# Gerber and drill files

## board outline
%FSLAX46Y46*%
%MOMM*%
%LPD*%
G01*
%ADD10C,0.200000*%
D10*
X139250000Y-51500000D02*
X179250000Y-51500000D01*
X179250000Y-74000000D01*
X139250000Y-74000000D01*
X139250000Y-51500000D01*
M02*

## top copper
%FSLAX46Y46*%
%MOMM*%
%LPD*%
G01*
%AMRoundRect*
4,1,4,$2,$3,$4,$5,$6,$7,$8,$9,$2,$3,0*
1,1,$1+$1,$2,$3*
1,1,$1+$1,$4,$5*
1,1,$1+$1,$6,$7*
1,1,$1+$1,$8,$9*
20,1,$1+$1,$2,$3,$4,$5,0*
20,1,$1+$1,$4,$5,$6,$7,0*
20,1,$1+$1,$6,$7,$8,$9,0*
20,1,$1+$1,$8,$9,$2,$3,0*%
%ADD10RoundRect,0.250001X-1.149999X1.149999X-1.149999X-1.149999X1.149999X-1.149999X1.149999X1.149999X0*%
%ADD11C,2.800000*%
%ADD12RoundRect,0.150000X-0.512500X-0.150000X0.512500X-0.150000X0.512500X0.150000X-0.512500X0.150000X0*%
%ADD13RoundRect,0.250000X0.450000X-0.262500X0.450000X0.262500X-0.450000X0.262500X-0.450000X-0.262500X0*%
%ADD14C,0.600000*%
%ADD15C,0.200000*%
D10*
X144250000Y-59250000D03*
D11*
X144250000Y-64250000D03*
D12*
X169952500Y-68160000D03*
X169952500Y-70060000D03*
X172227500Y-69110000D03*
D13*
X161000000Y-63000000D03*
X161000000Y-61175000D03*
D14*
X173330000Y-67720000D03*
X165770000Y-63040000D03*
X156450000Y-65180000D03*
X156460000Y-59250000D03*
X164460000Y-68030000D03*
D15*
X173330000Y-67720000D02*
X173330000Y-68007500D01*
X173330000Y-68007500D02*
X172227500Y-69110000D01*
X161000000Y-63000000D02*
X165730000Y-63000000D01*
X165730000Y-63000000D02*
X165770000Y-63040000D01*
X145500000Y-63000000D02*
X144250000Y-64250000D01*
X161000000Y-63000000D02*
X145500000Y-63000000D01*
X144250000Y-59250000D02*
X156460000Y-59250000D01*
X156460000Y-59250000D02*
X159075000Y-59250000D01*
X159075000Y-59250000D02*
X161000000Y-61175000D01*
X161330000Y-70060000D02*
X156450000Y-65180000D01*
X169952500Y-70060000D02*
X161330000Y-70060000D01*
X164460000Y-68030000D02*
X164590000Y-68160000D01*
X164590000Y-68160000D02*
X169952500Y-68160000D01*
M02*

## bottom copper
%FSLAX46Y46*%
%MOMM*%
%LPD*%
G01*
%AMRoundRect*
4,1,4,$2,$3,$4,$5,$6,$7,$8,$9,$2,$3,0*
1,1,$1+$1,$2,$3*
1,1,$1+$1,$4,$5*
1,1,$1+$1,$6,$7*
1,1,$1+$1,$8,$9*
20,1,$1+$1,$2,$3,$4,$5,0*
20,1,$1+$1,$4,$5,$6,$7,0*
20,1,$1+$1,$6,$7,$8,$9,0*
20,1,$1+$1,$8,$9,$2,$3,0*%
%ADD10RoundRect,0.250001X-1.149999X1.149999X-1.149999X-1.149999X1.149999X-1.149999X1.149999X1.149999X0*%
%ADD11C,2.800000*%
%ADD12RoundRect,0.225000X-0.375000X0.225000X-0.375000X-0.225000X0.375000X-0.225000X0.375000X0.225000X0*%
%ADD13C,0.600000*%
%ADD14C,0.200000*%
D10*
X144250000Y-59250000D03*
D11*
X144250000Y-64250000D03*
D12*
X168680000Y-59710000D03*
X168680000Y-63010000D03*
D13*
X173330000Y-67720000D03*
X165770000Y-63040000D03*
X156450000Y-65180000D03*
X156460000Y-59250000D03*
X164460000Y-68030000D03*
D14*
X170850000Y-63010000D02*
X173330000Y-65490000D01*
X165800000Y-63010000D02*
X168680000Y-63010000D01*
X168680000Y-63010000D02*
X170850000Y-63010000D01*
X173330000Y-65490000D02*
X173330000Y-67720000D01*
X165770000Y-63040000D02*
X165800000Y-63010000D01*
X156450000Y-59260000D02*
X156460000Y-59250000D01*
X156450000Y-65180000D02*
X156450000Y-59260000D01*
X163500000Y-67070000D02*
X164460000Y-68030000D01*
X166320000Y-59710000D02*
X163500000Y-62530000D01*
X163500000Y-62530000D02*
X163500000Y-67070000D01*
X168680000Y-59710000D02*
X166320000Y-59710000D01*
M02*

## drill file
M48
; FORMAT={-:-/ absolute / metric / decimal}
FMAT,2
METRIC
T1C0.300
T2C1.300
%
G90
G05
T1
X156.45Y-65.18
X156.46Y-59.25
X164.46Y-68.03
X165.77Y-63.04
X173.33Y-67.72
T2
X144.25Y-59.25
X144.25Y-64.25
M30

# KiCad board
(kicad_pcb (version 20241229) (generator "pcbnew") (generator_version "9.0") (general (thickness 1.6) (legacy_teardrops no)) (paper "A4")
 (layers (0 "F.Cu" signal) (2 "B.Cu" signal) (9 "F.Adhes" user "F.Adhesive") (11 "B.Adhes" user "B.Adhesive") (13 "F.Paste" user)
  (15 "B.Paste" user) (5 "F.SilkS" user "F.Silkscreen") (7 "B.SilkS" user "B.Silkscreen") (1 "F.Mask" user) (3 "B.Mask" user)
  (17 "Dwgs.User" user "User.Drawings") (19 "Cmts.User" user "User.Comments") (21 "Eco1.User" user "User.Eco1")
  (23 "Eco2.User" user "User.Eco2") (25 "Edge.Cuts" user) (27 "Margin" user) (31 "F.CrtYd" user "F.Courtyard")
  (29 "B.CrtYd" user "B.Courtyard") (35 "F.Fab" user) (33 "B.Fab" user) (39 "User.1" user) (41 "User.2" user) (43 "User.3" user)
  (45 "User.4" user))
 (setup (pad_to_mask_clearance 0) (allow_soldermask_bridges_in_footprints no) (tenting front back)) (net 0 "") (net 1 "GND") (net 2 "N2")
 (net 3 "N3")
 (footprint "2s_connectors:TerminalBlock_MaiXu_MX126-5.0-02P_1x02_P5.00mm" (layer "F.Cu") (at 144.25 59.25 -90)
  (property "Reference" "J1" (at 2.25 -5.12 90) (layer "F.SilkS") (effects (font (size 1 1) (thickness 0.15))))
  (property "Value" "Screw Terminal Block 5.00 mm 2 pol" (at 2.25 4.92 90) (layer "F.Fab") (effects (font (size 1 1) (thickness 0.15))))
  (pad "1" thru_hole roundrect (at 0 0 270) (size 2.8 2.8) (drill 1.3) (layers "*.Cu" "*.Mask") (remove_unused_layers no)
   (roundrect_rratio 0.089286) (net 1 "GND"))
  (pad "2" thru_hole circle (at 5 0 270) (size 2.8 2.8) (drill 1.3) (layers "*.Cu" "*.Mask") (remove_unused_layers no) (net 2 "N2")))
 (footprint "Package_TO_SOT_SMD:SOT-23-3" (layer "F.Cu") (at 171.09 69.11)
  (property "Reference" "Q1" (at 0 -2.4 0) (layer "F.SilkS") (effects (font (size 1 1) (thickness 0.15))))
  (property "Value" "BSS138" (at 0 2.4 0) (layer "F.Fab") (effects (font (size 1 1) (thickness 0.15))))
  (pad "1" smd roundrect (at -1.1375 -0.95) (size 1.325 0.6) (layers "F.Cu" "F.Mask" "F.Paste") (roundrect_rratio 0.25) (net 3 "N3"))
  (pad "2" smd roundrect (at -1.1375 0.95) (size 1.325 0.6) (layers "F.Cu" "F.Mask" "F.Paste") (roundrect_rratio 0.25) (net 1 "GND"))
  (pad "3" smd roundrect (at 1.1375 0) (size 1.325 0.6) (layers "F.Cu" "F.Mask" "F.Paste") (roundrect_rratio 0.25) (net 2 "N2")))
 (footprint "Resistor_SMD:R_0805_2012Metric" (layer "F.Cu") (at 161 62.0875 90)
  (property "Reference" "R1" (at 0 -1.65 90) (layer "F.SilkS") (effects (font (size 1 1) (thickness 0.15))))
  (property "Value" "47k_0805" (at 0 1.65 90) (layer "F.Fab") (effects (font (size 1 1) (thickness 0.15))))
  (pad "1" smd roundrect (at -0.9125 0 90) (size 1.025 1.4) (layers "F.Cu" "F.Mask" "F.Paste") (roundrect_rratio 0.243902) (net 2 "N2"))
  (pad "2" smd roundrect (at 0.9125 0 90) (size 1.025 1.4) (layers "F.Cu" "F.Mask" "F.Paste") (roundrect_rratio 0.243902) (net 1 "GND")))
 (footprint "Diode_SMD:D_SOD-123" (layer "B.Cu") (at 168.68 61.36 -90)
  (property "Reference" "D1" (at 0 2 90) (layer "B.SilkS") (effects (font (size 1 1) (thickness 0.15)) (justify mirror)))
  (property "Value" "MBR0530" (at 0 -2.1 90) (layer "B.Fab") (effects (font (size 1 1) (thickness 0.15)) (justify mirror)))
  (pad "1" smd roundrect (at -1.65 0 270) (size 0.9 1.2) (layers "B.Cu" "B.Mask" "B.Paste") (roundrect_rratio 0.25) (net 3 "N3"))
  (pad "2" smd roundrect (at 1.65 0 270) (size 0.9 1.2) (layers "B.Cu" "B.Mask" "B.Paste") (roundrect_rratio 0.25) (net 2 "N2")))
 (gr_rect (start 139.25 51.5) (end 179.25 74) (stroke (width 0.2) (type default)) (fill no) (layer "Edge.Cuts"))
 (segment (start 173.33 67.72) (end 173.33 68.0075) (width 0.2) (layer "F.Cu") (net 2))
 (segment (start 173.33 68.0075) (end 172.2275 69.11) (width 0.2) (layer "F.Cu") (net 2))
 (segment (start 161 63) (end 165.73 63) (width 0.2) (layer "F.Cu") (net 2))
 (segment (start 165.73 63) (end 165.77 63.04) (width 0.2) (layer "F.Cu") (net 2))
 (segment (start 145.5 63) (end 144.25 64.25) (width 0.2) (layer "F.Cu") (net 2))
 (segment (start 161 63) (end 145.5 63) (width 0.2) (layer "F.Cu") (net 2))
 (via (at 173.33 67.72) (size 0.6) (drill 0.3) (layers "F.Cu" "B.Cu") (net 2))
 (via (at 165.77 63.04) (size 0.6) (drill 0.3) (layers "F.Cu" "B.Cu") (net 2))
 (segment (start 170.85 63.01) (end 173.33 65.49) (width 0.2) (layer "B.Cu") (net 2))
 (segment (start 165.8 63.01) (end 168.68 63.01) (width 0.2) (layer "B.Cu") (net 2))
 (segment (start 168.68 63.01) (end 170.85 63.01) (width 0.2) (layer "B.Cu") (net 2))
 (segment (start 173.33 65.49) (end 173.33 67.72) (width 0.2) (layer "B.Cu") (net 2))
 (segment (start 165.77 63.04) (end 165.8 63.01) (width 0.2) (layer "B.Cu") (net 2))
 (segment (start 144.25 59.25) (end 156.46 59.25) (width 0.2) (layer "F.Cu") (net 1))
 (segment (start 156.46 59.25) (end 159.075 59.25) (width 0.2) (layer "F.Cu") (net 1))
 (segment (start 159.075 59.25) (end 161 61.175) (width 0.2) (layer "F.Cu") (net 1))
 (segment (start 161.33 70.06) (end 156.45 65.18) (width 0.2) (layer "F.Cu") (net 1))
 (segment (start 169.9525 70.06) (end 161.33 70.06) (width 0.2) (layer "F.Cu") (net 1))
 (via (at 156.45 65.18) (size 0.6) (drill 0.3) (layers "F.Cu" "B.Cu") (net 1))
 (via (at 156.46 59.25) (size 0.6) (drill 0.3) (layers "F.Cu" "B.Cu") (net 1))
 (segment (start 156.45 59.26) (end 156.46 59.25) (width 0.2) (layer "B.Cu") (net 1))
 (segment (start 156.45 65.18) (end 156.45 59.26) (width 0.2) (layer "B.Cu") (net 1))
 (segment (start 164.46 68.03) (end 164.59 68.16) (width 0.2) (layer "F.Cu") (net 3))
 (segment (start 164.59 68.16) (end 169.9525 68.16) (width 0.2) (layer "F.Cu") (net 3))
 (via (at 164.46 68.03) (size 0.6) (drill 0.3) (layers "F.Cu" "B.Cu") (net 3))
 (segment (start 163.5 67.07) (end 164.46 68.03) (width 0.2) (layer "B.Cu") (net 3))
 (segment (start 166.32 59.71) (end 163.5 62.53) (width 0.2) (layer "B.Cu") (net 3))
 (segment (start 163.5 62.53) (end 163.5 67.07) (width 0.2) (layer "B.Cu") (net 3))
 (segment (start 168.68 59.71) (end 166.32 59.71) (width 0.2) (layer "B.Cu") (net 3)))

